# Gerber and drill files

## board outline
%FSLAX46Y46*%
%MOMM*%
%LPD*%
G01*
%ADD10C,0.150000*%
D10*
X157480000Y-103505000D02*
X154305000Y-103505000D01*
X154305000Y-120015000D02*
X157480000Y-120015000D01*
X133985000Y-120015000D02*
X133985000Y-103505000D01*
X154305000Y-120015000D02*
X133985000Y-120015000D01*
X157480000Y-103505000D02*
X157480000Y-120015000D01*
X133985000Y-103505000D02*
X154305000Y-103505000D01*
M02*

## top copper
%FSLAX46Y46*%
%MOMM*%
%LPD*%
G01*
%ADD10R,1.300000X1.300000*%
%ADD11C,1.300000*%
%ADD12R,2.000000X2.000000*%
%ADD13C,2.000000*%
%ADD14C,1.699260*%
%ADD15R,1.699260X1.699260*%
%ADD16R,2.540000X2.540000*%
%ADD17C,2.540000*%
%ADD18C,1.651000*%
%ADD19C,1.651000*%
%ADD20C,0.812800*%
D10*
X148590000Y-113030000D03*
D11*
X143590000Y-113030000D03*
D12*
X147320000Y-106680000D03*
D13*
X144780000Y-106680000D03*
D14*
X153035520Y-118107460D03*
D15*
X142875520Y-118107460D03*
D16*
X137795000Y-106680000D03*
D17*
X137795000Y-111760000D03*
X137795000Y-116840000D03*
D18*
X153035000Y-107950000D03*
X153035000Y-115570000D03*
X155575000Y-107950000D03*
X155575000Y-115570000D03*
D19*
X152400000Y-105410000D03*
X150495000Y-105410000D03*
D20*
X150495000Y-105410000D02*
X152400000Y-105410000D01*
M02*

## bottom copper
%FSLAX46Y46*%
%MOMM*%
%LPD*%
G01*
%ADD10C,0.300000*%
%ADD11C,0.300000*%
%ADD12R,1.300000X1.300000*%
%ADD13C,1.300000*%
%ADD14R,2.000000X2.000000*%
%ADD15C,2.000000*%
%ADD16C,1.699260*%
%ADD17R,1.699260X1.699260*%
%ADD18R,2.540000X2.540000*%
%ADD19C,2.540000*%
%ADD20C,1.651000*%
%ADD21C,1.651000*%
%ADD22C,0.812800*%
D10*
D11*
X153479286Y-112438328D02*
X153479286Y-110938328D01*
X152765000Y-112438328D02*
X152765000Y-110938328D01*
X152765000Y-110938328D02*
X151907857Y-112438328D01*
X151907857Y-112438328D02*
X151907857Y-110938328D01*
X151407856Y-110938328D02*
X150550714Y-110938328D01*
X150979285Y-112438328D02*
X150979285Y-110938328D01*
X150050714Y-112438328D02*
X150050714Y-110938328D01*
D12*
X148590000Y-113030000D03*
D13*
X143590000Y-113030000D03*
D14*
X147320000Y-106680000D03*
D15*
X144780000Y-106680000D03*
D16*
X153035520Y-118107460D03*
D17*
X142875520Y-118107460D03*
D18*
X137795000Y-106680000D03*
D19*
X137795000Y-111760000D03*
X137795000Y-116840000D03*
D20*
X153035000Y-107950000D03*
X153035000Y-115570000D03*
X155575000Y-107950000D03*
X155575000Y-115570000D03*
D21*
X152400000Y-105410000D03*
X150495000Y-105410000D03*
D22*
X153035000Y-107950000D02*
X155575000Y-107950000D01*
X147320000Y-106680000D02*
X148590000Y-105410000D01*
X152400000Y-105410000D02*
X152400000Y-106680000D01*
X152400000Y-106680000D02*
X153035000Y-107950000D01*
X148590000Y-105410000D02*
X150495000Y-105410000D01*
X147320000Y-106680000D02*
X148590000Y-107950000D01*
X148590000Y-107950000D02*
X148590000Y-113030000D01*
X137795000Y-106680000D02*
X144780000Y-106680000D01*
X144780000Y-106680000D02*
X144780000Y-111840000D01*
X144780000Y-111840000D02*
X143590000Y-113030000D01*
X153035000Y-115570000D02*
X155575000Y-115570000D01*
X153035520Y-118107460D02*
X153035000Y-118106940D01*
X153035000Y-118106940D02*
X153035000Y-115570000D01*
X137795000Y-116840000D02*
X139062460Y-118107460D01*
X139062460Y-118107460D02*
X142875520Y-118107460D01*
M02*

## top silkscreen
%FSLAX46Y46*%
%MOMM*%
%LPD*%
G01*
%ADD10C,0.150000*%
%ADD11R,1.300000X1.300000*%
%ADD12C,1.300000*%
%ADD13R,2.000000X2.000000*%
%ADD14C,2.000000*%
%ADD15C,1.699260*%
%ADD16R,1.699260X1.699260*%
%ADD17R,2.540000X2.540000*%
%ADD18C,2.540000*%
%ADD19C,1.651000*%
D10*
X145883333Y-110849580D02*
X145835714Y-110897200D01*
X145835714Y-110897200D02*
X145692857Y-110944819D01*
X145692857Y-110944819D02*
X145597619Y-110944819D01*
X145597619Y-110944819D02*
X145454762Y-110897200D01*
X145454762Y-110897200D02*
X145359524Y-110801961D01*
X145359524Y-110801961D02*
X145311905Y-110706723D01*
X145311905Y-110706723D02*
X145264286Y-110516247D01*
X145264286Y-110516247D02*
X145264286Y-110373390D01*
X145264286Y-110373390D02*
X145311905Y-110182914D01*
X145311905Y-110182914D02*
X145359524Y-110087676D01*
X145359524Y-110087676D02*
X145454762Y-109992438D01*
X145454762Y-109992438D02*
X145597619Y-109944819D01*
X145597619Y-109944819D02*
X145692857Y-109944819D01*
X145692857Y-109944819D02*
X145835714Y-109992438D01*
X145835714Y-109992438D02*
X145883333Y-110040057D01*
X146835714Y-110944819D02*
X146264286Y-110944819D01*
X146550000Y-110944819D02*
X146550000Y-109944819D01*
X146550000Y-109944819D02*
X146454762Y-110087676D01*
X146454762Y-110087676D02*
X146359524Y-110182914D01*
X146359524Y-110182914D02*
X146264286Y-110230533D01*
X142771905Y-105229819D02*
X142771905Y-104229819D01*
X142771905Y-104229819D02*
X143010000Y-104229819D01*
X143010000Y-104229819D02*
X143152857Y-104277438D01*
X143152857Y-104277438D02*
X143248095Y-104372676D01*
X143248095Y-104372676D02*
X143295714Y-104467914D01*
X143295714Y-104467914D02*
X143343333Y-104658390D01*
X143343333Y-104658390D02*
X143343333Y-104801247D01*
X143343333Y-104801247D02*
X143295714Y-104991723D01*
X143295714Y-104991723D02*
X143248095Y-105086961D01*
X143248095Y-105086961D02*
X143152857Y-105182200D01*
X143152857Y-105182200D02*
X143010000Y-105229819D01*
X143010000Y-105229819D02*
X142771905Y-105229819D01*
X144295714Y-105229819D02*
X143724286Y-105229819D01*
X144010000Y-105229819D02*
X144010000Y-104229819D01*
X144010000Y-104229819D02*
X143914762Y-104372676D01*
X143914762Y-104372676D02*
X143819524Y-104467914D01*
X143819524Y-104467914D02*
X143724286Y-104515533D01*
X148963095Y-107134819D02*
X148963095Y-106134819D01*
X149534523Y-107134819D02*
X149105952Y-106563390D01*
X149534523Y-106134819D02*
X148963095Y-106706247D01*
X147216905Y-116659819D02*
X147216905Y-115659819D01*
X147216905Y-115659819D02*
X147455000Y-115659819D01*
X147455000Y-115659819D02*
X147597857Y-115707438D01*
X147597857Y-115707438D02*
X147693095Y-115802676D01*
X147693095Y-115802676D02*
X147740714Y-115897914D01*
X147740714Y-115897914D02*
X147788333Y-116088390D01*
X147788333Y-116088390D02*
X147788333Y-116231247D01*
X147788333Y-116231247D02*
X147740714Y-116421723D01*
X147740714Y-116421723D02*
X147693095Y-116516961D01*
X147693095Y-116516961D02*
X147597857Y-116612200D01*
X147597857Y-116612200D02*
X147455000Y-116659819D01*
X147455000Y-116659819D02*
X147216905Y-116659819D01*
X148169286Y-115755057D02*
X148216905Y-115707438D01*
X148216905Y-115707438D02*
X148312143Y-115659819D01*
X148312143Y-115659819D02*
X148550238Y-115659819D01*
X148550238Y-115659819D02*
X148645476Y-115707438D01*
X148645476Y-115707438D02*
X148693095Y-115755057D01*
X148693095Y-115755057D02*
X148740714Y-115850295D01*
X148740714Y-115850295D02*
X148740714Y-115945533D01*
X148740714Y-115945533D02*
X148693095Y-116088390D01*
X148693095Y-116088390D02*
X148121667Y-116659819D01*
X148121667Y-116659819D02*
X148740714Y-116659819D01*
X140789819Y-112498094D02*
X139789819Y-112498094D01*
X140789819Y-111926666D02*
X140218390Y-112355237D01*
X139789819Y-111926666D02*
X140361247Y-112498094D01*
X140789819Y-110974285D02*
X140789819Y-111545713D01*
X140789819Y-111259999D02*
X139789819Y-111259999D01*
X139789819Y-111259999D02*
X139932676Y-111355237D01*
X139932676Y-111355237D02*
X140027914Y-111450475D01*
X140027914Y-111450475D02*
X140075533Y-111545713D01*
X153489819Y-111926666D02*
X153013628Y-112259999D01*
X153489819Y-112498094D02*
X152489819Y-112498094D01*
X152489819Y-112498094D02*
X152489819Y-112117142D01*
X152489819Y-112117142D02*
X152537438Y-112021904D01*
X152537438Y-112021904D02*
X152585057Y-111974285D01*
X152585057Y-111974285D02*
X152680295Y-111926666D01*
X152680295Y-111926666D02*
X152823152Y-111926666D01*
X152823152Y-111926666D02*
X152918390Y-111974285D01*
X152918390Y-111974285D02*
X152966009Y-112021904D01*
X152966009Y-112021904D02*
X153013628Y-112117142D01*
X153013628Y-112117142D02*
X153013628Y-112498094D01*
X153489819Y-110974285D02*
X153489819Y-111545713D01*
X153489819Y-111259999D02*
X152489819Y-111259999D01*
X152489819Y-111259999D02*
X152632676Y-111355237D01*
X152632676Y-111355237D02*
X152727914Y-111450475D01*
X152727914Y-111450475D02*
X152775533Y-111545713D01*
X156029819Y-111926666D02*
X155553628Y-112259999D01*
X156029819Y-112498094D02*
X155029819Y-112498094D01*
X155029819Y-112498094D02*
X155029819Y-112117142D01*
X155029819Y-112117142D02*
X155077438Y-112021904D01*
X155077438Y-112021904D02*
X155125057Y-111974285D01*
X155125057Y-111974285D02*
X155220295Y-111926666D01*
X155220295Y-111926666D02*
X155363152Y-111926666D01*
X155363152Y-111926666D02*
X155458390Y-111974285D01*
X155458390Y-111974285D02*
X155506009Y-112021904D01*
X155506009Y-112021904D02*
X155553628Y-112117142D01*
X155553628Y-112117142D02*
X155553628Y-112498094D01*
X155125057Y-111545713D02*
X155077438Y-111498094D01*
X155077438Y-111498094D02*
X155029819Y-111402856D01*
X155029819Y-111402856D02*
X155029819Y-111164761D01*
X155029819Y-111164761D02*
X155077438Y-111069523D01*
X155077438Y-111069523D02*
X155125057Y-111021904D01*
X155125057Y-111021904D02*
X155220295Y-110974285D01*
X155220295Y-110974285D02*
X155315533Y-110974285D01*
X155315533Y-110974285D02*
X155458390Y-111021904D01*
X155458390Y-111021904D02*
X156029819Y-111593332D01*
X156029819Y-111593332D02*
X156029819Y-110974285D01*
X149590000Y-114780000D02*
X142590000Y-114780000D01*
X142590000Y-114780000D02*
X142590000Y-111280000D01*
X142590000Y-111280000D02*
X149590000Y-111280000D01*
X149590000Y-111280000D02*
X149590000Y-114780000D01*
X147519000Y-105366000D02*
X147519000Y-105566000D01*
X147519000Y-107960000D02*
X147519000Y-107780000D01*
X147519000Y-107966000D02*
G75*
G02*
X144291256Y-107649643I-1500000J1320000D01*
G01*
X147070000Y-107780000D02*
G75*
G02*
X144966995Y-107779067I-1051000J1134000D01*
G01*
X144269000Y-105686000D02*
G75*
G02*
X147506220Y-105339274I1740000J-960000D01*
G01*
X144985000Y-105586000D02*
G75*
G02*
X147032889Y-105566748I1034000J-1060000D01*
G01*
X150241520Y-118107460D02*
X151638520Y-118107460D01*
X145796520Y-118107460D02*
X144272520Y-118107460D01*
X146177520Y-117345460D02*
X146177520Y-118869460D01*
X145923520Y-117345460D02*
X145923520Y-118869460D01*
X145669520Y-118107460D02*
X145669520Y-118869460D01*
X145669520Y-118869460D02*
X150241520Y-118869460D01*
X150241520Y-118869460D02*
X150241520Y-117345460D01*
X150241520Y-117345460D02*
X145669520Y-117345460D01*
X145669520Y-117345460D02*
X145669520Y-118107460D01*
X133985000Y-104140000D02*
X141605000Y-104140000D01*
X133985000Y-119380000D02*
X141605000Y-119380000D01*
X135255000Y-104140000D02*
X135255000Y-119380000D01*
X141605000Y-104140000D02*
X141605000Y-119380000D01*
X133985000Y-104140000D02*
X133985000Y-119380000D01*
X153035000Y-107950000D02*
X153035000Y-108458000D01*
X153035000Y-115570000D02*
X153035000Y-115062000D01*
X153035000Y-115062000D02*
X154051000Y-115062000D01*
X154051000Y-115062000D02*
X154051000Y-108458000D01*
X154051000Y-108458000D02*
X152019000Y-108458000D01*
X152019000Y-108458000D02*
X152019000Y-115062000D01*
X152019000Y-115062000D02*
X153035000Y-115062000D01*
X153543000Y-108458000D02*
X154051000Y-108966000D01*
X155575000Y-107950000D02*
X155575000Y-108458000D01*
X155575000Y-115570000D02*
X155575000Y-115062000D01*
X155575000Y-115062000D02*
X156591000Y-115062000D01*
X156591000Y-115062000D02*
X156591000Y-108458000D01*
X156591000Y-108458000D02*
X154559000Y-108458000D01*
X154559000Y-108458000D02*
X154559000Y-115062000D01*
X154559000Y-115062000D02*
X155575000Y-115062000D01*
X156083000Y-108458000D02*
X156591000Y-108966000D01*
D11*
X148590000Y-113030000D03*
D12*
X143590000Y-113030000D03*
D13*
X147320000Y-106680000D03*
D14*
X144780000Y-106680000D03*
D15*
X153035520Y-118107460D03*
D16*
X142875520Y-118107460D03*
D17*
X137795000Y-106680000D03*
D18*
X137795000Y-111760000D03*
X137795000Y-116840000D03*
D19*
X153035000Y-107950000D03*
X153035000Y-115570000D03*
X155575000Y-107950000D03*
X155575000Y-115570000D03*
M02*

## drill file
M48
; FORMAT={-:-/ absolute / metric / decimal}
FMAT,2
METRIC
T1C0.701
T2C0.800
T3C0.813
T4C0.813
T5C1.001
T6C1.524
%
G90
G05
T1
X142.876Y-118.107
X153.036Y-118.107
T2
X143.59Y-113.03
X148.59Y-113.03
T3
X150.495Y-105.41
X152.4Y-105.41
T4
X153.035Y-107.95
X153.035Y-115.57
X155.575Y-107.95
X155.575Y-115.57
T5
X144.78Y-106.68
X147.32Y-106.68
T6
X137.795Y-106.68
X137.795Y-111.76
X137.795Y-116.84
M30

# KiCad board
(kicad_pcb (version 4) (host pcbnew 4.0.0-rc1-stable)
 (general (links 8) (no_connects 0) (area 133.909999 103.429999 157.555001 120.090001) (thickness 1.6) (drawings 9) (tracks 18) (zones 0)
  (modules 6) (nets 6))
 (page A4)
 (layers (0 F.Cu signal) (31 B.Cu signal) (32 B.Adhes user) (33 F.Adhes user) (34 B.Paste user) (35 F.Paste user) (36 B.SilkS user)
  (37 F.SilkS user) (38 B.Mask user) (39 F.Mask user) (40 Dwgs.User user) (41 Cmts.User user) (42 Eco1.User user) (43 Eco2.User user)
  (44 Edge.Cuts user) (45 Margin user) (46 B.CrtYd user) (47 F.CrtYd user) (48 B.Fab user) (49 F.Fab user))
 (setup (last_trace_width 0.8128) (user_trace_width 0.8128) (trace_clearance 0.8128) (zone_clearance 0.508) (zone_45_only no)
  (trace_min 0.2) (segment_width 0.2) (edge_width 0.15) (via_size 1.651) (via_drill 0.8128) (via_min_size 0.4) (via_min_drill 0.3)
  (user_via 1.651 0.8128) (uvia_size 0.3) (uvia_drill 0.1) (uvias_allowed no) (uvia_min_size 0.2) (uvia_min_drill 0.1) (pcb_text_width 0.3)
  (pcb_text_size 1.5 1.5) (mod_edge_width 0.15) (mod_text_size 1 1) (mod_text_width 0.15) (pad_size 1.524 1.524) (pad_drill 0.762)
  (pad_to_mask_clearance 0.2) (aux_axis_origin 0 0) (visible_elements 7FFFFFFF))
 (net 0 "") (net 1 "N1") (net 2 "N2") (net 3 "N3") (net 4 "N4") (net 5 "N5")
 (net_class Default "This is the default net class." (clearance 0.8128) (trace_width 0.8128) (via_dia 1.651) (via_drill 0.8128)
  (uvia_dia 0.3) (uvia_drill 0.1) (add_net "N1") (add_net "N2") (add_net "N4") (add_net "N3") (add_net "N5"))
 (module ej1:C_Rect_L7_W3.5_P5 (layer F.Cu) (at 148.59 113.03 180)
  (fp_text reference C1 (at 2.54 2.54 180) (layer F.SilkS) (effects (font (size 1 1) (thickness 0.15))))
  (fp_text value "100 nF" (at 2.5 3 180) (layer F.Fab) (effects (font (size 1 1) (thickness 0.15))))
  (fp_line (start -1 -1.75) (end 6 -1.75) (layer F.SilkS) (width 0.15))
  (fp_line (start 6 -1.75) (end 6 1.75) (layer F.SilkS) (width 0.15))
  (fp_line (start 6 1.75) (end -1 1.75) (layer F.SilkS) (width 0.15))
  (fp_line (start -1 1.75) (end -1 -1.75) (layer F.SilkS) (width 0.15))
  (pad 1 thru_hole rect (at 0 0 180) (size 1.3 1.3) (drill 0.8) (layers *.Cu *.Mask F.SilkS) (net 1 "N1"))
  (pad 2 thru_hole circle (at 5 0 180) (size 1.3 1.3) (drill 0.8) (layers *.Cu *.Mask F.SilkS) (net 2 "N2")))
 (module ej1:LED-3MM (layer F.Cu) (at 147.32 106.68 180)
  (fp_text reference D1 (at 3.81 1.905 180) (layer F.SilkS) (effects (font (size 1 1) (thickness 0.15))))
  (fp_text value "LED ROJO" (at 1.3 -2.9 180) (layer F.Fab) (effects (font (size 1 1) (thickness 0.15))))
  (fp_line (start -0.199 1.314) (end -0.199 1.114) (layer F.SilkS) (width 0.15))
  (fp_line (start -0.199 -1.28) (end -0.199 -1.1) (layer F.SilkS) (width 0.15))
  (fp_arc (start 1.301 0.034) (end -0.199 -1.286) (angle 108.5) (layer F.SilkS) (width 0.15))
  (fp_arc (start 1.301 0.034) (end 0.25 -1.1) (angle 85.7) (layer F.SilkS) (width 0.15))
  (fp_arc (start 1.311 0.034) (end 3.051 0.994) (angle 110) (layer F.SilkS) (width 0.15))
  (fp_arc (start 1.301 0.034) (end 2.335 1.094) (angle 87.5) (layer F.SilkS) (width 0.15))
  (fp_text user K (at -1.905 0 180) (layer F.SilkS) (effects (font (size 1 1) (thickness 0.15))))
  (pad 1 thru_hole rect (at 0 0 270) (size 2 2) (drill 1.00076) (layers *.Cu *.Mask F.SilkS) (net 1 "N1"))
  (pad 2 thru_hole circle (at 2.54 0 180) (size 2 2) (drill 1.00076) (layers *.Cu *.Mask F.SilkS) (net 2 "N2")))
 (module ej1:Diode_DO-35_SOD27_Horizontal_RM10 (layer F.Cu) (at 142.875 118.11)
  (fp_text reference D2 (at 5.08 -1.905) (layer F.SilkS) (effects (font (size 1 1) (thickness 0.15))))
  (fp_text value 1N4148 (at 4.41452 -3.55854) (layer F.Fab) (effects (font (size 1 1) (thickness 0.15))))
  (fp_line (start 7.36652 -0.00254) (end 8.76352 -0.00254) (layer F.SilkS) (width 0.15))
  (fp_line (start 2.92152 -0.00254) (end 1.39752 -0.00254) (layer F.SilkS) (width 0.15))
  (fp_line (start 3.30252 -0.76454) (end 3.30252 0.75946) (layer F.SilkS) (width 0.15))
  (fp_line (start 3.04852 -0.76454) (end 3.04852 0.75946) (layer F.SilkS) (width 0.15))
  (fp_line (start 2.79452 -0.00254) (end 2.79452 0.75946) (layer F.SilkS) (width 0.15))
  (fp_line (start 2.79452 0.75946) (end 7.36652 0.75946) (layer F.SilkS) (width 0.15))
  (fp_line (start 7.36652 0.75946) (end 7.36652 -0.76454) (layer F.SilkS) (width 0.15))
  (fp_line (start 7.36652 -0.76454) (end 2.79452 -0.76454) (layer F.SilkS) (width 0.15))
  (fp_line (start 2.79452 -0.76454) (end 2.79452 -0.00254) (layer F.SilkS) (width 0.15))
  (pad 2 thru_hole circle (at 10.16052 -0.00254 180) (size 1.69926 1.69926) (drill 0.70104) (layers *.Cu *.Mask F.SilkS) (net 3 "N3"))
  (pad 1 thru_hole rect (at 0.00052 -0.00254 180) (size 1.69926 1.69926) (drill 0.70104) (layers *.Cu *.Mask F.SilkS) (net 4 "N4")))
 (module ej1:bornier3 (layer F.Cu) (at 137.795 111.76 270)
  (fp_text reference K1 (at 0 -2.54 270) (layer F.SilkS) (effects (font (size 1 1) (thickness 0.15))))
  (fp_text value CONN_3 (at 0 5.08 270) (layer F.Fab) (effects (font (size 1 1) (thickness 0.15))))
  (fp_line (start -7.62 3.81) (end -7.62 -3.81) (layer F.SilkS) (width 0.15))
  (fp_line (start 7.62 3.81) (end 7.62 -3.81) (layer F.SilkS) (width 0.15))
  (fp_line (start -7.62 2.54) (end 7.62 2.54) (layer F.SilkS) (width 0.15))
  (fp_line (start -7.62 -3.81) (end 7.62 -3.81) (layer F.SilkS) (width 0.15))
  (fp_line (start -7.62 3.81) (end 7.62 3.81) (layer F.SilkS) (width 0.15))
  (pad 1 thru_hole rect (at -5.08 0 270) (size 2.54 2.54) (drill 1.524) (layers *.Cu *.Mask F.SilkS) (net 2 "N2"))
  (pad 2 thru_hole circle (at 0 0 270) (size 2.54 2.54) (drill 1.524) (layers *.Cu *.Mask F.SilkS) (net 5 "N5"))
  (pad 3 thru_hole circle (at 5.08 0 270) (size 2.54 2.54) (drill 1.524) (layers *.Cu *.Mask F.SilkS) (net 4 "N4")))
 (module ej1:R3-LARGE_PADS (layer F.Cu) (at 153.035 111.76 270)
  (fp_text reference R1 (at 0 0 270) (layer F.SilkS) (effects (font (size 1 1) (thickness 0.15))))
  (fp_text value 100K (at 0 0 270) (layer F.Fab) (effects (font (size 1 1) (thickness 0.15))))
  (fp_line (start -3.81 0) (end -3.302 0) (layer F.SilkS) (width 0.15))
  (fp_line (start 3.81 0) (end 3.302 0) (layer F.SilkS) (width 0.15))
  (fp_line (start 3.302 0) (end 3.302 -1.016) (layer F.SilkS) (width 0.15))
  (fp_line (start 3.302 -1.016) (end -3.302 -1.016) (layer F.SilkS) (width 0.15))
  (fp_line (start -3.302 -1.016) (end -3.302 1.016) (layer F.SilkS) (width 0.15))
  (fp_line (start -3.302 1.016) (end 3.302 1.016) (layer F.SilkS) (width 0.15))
  (fp_line (start 3.302 1.016) (end 3.302 0) (layer F.SilkS) (width 0.15))
  (fp_line (start -3.302 -0.508) (end -2.794 -1.016) (layer F.SilkS) (width 0.15))
  (pad 1 thru_hole circle (at -3.81 0 270) (size 1.651 1.651) (drill 0.8128) (layers *.Cu *.Mask F.SilkS) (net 1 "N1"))
  (pad 2 thru_hole circle (at 3.81 0 270) (size 1.651 1.651) (drill 0.8128) (layers *.Cu *.Mask F.SilkS) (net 3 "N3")))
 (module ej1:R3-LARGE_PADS (layer F.Cu) (at 155.575 111.76 270)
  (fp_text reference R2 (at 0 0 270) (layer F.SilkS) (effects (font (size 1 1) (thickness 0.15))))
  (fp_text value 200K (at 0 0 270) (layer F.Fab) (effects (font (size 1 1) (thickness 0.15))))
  (fp_line (start -3.81 0) (end -3.302 0) (layer F.SilkS) (width 0.15))
  (fp_line (start 3.81 0) (end 3.302 0) (layer F.SilkS) (width 0.15))
  (fp_line (start 3.302 0) (end 3.302 -1.016) (layer F.SilkS) (width 0.15))
  (fp_line (start 3.302 -1.016) (end -3.302 -1.016) (layer F.SilkS) (width 0.15))
  (fp_line (start -3.302 -1.016) (end -3.302 1.016) (layer F.SilkS) (width 0.15))
  (fp_line (start -3.302 1.016) (end 3.302 1.016) (layer F.SilkS) (width 0.15))
  (fp_line (start 3.302 1.016) (end 3.302 0) (layer F.SilkS) (width 0.15))
  (fp_line (start -3.302 -0.508) (end -2.794 -1.016) (layer F.SilkS) (width 0.15))
  (pad 1 thru_hole circle (at -3.81 0 270) (size 1.651 1.651) (drill 0.8128) (layers *.Cu *.Mask F.SilkS) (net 1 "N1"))
  (pad 2 thru_hole circle (at 3.81 0 270) (size 1.651 1.651) (drill 0.8128) (layers *.Cu *.Mask F.SilkS) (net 3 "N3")))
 (gr_line (start 157.48 103.505) (end 154.305 103.505) (angle 90) (layer Edge.Cuts) (width 0.15))
 (gr_line (start 154.305 120.015) (end 157.48 120.015) (angle 90) (layer Edge.Cuts) (width 0.15))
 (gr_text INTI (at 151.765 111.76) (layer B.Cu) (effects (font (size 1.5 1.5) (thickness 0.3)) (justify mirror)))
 (gr_line (start 133.985 120.015) (end 133.985 103.505) (angle 90) (layer Edge.Cuts) (width 0.15))
 (gr_line (start 154.305 120.015) (end 133.985 120.015) (angle 90) (layer Edge.Cuts) (width 0.15))
 (gr_line (start 157.48 103.505) (end 157.48 120.015) (angle 90) (layer Edge.Cuts) (width 0.15))
 (gr_line (start 133.985 103.505) (end 154.305 103.505) (angle 90) (layer Edge.Cuts) (width 0.15))
 (segment (start 153.035 107.95) (end 155.575 107.95) (width 0.8128) (layer B.Cu) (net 1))
 (segment (start 147.32 106.68) (end 148.59 105.41) (width 0.8128) (layer B.Cu) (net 1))
 (segment (start 152.4 105.41) (end 152.4 106.68) (width 0.8128) (layer B.Cu) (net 1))
 (segment (start 152.4 106.68) (end 153.035 107.95) (width 0.8128) (layer B.Cu) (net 1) (status 20))
 (via (at 152.4 105.41) (size 1.651) (drill 0.8128) (layers F.Cu B.Cu) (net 1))
 (segment (start 150.495 105.41) (end 152.4 105.41) (width 0.8128) (layer F.Cu) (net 1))
 (via (at 150.495 105.41) (size 1.651) (drill 0.8128) (layers F.Cu B.Cu) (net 1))
 (segment (start 148.59 105.41) (end 150.495 105.41) (width 0.8128) (layer B.Cu) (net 1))
 (segment (start 147.32 106.68) (end 148.59 107.95) (width 0.8128) (layer B.Cu) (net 1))
 (segment (start 148.59 107.95) (end 148.59 113.03) (width 0.8128) (layer B.Cu) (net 1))
 (segment (start 137.795 106.68) (end 144.78 106.68) (width 0.8128) (layer B.Cu) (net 2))
 (segment (start 144.78 106.68) (end 144.78 111.84) (width 0.8128) (layer B.Cu) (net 2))
 (segment (start 144.78 111.84) (end 143.59 113.03) (width 0.8128) (layer B.Cu) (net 2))
 (segment (start 153.035 115.57) (end 155.575 115.57) (width 0.8128) (layer B.Cu) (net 3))
 (segment (start 153.03552 118.10746) (end 153.035 118.10694) (width 0.8128) (layer B.Cu) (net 3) (status 30))
 (segment (start 153.035 118.10694) (end 153.035 115.57) (width 0.8128) (layer B.Cu) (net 3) (status 10))
 (segment (start 137.795 116.84) (end 139.06246 118.10746) (width 0.8128) (layer B.Cu) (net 4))
 (segment (start 139.06246 118.10746) (end 142.87552 118.10746) (width 0.8128) (layer B.Cu) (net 4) (status 20)))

